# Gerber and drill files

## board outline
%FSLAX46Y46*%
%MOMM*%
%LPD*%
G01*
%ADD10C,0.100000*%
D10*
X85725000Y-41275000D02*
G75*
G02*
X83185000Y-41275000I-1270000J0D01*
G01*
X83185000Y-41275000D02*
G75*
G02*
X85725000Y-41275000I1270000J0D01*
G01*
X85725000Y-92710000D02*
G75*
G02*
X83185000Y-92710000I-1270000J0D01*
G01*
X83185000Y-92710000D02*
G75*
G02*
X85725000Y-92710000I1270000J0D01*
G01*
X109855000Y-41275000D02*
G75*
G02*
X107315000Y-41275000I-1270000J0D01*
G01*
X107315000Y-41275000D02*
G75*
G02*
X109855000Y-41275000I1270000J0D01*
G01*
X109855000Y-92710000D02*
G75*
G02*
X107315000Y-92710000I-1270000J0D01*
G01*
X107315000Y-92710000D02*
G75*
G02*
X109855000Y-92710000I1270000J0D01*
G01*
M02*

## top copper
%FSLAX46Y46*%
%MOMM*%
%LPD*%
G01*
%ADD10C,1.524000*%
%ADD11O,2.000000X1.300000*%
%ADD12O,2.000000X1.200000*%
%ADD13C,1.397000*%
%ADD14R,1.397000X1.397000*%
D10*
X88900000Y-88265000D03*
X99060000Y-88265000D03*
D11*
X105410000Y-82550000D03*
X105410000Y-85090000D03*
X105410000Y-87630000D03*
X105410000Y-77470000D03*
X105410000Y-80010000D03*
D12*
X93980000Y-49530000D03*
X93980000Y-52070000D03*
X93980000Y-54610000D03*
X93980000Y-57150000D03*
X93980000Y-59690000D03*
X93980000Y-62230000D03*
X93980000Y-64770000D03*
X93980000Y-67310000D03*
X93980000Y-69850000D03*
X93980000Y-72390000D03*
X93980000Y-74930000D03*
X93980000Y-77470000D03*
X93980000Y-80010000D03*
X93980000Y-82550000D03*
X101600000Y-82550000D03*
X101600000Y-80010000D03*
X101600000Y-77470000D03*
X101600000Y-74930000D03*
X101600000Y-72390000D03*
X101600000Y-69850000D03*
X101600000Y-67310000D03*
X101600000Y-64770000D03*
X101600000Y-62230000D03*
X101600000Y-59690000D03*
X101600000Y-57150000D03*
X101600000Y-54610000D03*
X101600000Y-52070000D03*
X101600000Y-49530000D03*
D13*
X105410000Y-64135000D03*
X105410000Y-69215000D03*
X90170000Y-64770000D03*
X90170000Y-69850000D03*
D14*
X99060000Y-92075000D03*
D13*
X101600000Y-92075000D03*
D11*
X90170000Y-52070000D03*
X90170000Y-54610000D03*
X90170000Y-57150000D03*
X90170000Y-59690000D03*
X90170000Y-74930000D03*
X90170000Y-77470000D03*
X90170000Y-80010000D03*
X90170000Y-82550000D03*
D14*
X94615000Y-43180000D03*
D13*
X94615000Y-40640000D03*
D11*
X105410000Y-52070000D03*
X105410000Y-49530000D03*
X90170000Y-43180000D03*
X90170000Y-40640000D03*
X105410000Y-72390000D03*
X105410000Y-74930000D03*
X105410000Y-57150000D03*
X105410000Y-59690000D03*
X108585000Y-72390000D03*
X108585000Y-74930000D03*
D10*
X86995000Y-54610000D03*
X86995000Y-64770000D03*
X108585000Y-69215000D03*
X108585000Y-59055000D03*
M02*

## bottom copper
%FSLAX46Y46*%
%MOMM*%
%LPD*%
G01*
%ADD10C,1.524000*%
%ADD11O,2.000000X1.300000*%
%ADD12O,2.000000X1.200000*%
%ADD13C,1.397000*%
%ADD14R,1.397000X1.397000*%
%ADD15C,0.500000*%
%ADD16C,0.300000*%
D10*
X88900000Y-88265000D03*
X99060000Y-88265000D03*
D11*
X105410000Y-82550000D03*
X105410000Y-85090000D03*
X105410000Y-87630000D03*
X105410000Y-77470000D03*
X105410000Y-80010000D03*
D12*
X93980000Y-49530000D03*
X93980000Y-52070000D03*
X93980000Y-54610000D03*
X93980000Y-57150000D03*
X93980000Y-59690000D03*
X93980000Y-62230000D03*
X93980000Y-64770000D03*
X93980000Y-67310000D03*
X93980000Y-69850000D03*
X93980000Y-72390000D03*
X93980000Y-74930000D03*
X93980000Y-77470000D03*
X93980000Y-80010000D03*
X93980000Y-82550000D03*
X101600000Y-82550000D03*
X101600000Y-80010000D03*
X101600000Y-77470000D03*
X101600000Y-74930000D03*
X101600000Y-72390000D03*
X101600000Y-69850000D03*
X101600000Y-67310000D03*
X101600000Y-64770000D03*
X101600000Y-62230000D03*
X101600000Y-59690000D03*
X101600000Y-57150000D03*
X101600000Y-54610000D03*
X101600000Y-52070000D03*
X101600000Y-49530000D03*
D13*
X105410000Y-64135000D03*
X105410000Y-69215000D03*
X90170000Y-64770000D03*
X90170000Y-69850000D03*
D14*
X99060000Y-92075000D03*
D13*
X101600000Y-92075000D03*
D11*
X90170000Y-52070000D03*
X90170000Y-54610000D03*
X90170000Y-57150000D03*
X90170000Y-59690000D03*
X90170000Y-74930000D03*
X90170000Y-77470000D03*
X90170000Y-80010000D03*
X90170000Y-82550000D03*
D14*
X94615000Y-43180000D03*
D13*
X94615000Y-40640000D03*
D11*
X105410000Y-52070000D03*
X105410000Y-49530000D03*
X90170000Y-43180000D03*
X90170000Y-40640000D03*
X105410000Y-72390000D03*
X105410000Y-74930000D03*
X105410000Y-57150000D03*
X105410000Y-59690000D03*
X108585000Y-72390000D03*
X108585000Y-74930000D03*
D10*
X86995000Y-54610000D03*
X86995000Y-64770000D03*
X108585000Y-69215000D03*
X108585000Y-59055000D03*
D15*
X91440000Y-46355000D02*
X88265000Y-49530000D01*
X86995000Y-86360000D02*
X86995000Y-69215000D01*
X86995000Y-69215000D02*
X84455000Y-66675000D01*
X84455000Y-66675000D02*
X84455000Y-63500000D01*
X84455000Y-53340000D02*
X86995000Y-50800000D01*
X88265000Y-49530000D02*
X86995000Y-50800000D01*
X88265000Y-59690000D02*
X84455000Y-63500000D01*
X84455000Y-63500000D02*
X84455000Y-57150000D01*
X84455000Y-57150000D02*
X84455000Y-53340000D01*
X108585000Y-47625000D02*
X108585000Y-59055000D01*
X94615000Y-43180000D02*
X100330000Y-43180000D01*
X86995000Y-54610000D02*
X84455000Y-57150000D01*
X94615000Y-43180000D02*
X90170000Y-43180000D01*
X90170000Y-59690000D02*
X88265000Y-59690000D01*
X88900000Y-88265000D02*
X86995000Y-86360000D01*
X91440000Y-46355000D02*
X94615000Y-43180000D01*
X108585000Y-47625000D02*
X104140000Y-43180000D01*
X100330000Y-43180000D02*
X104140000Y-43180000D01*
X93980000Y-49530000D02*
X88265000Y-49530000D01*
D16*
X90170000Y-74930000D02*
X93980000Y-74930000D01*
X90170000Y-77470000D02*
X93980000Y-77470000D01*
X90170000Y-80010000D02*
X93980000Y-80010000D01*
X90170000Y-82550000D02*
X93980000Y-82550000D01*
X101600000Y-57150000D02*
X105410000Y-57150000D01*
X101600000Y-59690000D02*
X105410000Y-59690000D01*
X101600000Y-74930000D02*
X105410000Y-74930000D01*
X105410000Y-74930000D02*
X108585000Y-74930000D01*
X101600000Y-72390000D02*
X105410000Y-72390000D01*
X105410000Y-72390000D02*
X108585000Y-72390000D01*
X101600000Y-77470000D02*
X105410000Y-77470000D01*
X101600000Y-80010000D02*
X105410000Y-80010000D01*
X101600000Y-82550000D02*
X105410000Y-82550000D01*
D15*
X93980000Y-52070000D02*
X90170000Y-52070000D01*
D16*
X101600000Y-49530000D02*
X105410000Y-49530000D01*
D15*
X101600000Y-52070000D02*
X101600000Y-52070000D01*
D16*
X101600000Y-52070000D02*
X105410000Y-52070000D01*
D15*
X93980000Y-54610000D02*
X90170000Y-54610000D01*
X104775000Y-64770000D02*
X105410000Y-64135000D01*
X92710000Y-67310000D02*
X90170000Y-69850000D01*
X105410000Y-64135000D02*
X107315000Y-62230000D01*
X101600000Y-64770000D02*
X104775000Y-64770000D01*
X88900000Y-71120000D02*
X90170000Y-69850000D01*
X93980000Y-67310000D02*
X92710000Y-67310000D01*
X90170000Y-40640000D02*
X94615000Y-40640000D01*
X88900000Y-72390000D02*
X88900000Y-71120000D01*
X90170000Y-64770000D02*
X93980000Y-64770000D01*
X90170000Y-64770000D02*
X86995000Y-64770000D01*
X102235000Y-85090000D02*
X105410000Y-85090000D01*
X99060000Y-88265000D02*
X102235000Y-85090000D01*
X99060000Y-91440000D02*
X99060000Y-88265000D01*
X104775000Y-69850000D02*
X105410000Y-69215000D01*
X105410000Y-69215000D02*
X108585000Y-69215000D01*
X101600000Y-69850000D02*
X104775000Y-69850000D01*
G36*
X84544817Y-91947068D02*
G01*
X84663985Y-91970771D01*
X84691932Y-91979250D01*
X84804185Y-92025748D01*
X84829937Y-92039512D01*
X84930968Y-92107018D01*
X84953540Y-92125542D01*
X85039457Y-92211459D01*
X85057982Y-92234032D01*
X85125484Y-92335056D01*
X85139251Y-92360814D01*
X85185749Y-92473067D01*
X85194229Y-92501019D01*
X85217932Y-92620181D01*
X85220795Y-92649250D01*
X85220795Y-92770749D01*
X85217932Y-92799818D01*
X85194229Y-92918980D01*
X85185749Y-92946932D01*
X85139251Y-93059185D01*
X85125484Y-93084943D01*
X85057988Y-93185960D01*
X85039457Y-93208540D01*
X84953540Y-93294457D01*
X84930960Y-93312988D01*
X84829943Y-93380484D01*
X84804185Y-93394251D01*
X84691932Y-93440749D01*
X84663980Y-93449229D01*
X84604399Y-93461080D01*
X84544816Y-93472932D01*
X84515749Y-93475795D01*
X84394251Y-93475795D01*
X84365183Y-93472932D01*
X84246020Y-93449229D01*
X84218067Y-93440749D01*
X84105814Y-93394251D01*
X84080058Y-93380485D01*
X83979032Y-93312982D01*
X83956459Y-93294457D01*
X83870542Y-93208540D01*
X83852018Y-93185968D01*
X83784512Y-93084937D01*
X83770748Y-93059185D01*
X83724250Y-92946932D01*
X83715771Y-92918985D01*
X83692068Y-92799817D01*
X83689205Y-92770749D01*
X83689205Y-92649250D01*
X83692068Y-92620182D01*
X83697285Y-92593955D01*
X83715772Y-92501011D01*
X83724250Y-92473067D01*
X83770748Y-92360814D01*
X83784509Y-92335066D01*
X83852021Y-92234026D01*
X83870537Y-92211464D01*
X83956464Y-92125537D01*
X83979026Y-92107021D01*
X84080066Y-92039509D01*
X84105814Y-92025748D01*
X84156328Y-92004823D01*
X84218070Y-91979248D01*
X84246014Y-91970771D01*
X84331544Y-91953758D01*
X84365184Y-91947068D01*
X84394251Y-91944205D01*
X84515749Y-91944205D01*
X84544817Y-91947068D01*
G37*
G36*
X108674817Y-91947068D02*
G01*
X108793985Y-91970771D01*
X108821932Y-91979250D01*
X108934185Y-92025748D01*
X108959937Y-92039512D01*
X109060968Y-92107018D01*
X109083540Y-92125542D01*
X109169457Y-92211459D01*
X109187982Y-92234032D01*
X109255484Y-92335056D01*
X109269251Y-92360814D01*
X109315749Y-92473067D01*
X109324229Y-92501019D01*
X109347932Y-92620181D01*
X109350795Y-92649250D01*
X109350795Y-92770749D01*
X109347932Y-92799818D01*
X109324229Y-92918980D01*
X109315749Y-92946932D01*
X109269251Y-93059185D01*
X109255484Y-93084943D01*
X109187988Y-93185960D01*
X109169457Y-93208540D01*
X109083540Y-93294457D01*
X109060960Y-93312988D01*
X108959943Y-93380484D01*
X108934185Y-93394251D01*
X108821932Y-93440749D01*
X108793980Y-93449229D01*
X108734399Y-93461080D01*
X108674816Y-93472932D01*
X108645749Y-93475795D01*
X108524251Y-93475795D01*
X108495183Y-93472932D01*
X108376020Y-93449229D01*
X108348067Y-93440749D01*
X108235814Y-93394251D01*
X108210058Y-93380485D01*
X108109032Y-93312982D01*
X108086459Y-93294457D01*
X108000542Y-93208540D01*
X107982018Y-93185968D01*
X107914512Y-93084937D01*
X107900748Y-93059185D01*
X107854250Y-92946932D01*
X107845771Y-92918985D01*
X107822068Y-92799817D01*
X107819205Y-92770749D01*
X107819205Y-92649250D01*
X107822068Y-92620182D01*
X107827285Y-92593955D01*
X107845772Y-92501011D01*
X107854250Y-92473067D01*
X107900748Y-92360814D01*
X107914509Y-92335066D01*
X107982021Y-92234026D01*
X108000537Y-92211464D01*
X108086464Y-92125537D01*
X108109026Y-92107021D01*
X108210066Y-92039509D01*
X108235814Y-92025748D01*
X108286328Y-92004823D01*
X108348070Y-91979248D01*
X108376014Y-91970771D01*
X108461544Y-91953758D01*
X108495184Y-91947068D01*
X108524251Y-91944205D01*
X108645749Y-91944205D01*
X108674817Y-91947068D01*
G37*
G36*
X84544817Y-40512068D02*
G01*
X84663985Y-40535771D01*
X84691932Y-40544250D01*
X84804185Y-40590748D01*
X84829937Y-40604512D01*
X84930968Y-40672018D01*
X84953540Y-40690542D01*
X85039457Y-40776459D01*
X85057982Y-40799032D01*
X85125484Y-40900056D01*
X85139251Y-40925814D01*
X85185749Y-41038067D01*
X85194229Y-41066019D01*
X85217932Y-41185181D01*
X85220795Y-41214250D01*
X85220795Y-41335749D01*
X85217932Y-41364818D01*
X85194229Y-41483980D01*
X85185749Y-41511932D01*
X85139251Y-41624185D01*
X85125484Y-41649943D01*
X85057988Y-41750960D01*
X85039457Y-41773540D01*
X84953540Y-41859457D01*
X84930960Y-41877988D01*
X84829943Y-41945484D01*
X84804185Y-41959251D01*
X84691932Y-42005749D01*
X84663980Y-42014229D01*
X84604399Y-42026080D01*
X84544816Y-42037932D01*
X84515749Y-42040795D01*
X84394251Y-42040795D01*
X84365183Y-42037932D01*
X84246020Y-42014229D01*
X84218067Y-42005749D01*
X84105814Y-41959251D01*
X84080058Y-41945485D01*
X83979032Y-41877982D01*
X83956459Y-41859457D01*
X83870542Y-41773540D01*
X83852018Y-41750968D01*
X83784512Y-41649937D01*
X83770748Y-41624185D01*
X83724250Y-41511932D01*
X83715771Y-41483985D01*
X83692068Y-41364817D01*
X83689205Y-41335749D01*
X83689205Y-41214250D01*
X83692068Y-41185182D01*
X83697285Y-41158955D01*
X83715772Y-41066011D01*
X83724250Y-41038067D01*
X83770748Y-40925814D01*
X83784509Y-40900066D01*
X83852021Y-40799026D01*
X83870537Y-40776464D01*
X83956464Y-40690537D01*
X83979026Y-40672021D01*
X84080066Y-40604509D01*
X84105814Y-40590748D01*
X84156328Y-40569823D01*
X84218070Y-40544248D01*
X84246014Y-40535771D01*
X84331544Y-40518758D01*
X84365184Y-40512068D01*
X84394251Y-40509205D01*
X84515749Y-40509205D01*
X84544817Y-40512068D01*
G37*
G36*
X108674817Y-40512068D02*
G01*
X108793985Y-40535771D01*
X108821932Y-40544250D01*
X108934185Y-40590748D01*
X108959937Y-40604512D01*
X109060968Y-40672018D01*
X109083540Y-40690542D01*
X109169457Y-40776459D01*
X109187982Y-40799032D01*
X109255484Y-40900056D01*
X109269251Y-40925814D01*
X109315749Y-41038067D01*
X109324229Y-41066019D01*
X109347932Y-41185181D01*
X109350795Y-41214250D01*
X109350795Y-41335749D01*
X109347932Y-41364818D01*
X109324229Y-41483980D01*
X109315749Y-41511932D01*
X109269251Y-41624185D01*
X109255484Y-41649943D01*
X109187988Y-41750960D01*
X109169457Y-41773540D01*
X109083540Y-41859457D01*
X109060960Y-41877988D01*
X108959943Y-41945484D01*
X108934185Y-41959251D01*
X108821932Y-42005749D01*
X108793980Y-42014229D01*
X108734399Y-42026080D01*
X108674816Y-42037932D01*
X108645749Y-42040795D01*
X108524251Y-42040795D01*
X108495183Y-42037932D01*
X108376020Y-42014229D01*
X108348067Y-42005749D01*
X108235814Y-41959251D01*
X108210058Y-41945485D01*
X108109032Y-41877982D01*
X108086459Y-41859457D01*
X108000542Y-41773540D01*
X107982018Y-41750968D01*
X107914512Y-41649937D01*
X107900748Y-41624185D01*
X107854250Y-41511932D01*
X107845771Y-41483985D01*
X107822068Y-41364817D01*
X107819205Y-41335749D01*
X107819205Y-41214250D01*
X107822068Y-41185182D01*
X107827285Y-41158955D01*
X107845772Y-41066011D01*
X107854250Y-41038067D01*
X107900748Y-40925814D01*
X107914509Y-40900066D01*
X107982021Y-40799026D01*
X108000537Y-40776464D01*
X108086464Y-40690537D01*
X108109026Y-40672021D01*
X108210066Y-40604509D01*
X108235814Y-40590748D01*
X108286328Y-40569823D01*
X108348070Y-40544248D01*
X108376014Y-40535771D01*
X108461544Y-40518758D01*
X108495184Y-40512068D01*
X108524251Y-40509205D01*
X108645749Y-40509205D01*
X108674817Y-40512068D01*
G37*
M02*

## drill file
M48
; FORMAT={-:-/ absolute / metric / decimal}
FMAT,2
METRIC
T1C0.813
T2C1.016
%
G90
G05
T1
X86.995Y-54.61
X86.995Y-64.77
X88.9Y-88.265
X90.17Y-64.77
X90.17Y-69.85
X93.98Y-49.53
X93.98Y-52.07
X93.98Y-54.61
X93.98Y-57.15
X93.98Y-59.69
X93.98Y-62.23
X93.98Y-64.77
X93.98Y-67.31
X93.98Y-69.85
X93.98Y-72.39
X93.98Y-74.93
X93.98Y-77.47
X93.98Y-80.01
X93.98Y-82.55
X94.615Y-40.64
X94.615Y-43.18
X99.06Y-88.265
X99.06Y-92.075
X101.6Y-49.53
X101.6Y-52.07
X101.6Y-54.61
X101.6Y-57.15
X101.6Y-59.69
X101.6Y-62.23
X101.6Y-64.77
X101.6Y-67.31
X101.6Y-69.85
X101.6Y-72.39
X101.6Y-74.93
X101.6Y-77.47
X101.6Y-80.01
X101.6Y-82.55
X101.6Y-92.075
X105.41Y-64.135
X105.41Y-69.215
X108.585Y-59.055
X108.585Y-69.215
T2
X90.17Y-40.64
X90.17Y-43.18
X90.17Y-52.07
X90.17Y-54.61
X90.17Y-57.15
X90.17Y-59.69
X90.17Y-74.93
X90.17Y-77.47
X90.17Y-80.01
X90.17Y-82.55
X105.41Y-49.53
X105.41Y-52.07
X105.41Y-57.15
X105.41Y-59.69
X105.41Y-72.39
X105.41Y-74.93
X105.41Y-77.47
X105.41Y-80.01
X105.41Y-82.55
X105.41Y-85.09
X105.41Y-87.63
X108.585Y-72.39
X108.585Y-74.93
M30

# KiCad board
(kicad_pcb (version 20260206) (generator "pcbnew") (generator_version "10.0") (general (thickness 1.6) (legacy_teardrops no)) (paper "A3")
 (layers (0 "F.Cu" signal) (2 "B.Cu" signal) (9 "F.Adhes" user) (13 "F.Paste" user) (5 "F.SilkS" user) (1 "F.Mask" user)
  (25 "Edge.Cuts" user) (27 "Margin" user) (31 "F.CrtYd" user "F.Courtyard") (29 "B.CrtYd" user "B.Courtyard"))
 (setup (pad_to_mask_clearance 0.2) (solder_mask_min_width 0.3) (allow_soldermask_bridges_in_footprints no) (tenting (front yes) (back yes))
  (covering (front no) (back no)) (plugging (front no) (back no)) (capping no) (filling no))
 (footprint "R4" (layer "F.Cu") (at 93.98 88.265)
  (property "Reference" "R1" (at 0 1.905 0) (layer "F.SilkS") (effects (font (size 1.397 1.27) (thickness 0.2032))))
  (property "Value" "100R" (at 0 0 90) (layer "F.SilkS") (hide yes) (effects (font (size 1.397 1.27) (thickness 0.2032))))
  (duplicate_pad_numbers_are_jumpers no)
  (pad "1" thru_hole circle (at -5.08 0) (size 1.524 1.524) (drill 0.8128) (layers "*.Cu" "*.Mask" "F.SilkS") (remove_unused_layers no)
   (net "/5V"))
  (pad "2" thru_hole circle (at 5.08 0) (size 1.524 1.524) (drill 0.8128) (layers "*.Cu" "*.Mask" "F.SilkS") (remove_unused_layers no)
   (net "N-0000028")))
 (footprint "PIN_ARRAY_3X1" (layer "F.Cu") (at 105.41 85.09 -90)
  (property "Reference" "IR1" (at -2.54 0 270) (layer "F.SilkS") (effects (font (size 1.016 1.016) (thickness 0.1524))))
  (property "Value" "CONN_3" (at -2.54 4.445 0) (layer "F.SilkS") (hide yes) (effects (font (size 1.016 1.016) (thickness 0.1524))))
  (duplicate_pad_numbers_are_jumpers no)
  (pad "1" thru_hole oval (at -2.54 0 270) (size 1.3 2) (drill 1.016) (layers "*.Cu" "*.Mask" "F.SilkS") (remove_unused_layers no)
   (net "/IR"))
  (pad "2" thru_hole oval (at 0 0 270) (size 1.3 2) (drill 1.016) (layers "*.Cu" "*.Mask" "F.SilkS") (remove_unused_layers no)
   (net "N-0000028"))
  (pad "3" thru_hole oval (at 2.54 0 270) (size 1.3 2) (drill 1.016) (layers "*.Cu" "*.Mask" "F.SilkS") (remove_unused_layers no)
   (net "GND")))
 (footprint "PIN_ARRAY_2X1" (layer "F.Cu") (at 105.41 78.74 -90)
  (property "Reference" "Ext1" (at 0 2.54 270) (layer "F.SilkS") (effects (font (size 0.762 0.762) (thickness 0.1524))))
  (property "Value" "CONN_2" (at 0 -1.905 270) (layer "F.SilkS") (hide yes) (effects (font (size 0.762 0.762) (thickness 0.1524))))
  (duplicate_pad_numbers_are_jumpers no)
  (pad "1" thru_hole oval (at -1.27 0 270) (size 1.3 2) (drill 1.016) (layers "*.Cu" "*.Mask" "F.SilkS") (remove_unused_layers no)
   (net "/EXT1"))
  (pad "2" thru_hole oval (at 1.27 0 270) (size 1.3 2) (drill 1.016) (layers "*.Cu" "*.Mask" "F.SilkS") (remove_unused_layers no)
   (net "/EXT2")))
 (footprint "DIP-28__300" (layer "F.Cu") (at 97.79 66.04 -90)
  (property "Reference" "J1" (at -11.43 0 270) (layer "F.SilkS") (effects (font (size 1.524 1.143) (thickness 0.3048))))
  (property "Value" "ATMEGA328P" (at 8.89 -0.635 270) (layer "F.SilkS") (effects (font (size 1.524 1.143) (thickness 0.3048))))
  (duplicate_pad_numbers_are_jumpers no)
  (pad "1" thru_hole oval (at -16.51 3.81 270) (size 1.2 2) (drill 0.8128) (layers "*.Cu" "*.Mask" "F.SilkS") (remove_unused_layers no)
   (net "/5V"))
  (pad "2" thru_hole oval (at -13.97 3.81 270) (size 1.2 2) (drill 0.8128) (layers "*.Cu" "*.Mask" "F.SilkS") (remove_unused_layers no)
   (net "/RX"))
  (pad "3" thru_hole oval (at -11.43 3.81 270) (size 1.2 2) (drill 0.8128) (layers "*.Cu" "*.Mask" "F.SilkS") (remove_unused_layers no)
   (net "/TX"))
  (pad "4" thru_hole oval (at -8.89 3.81 270) (size 1.2 2) (drill 0.8128) (layers "*.Cu" "*.Mask" "F.SilkS") (remove_unused_layers no))
  (pad "5" thru_hole oval (at -6.35 3.81 270) (size 1.2 2) (drill 0.8128) (layers "*.Cu" "*.Mask" "F.SilkS") (remove_unused_layers no))
  (pad "6" thru_hole oval (at -3.81 3.81 270) (size 1.2 2) (drill 0.8128) (layers "*.Cu" "*.Mask" "F.SilkS") (remove_unused_layers no))
  (pad "7" thru_hole oval (at -1.27 3.81 270) (size 1.2 2) (drill 0.8128) (layers "*.Cu" "*.Mask" "F.SilkS") (remove_unused_layers no)
   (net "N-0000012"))
  (pad "8" thru_hole oval (at 1.27 3.81 270) (size 1.2 2) (drill 0.8128) (layers "*.Cu" "*.Mask" "F.SilkS") (remove_unused_layers no)
   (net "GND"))
  (pad "9" thru_hole oval (at 3.81 3.81 270) (size 1.2 2) (drill 0.8128) (layers "*.Cu" "*.Mask" "F.SilkS") (remove_unused_layers no))
  (pad "10" thru_hole oval (at 6.35 3.81 270) (size 1.2 2) (drill 0.8128) (layers "*.Cu" "*.Mask" "F.SilkS") (remove_unused_layers no))
  (pad "11" thru_hole oval (at 8.89 3.81 270) (size 1.2 2) (drill 0.8128) (layers "*.Cu" "*.Mask" "F.SilkS") (remove_unused_layers no)
   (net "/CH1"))
  (pad "12" thru_hole oval (at 11.43 3.81 270) (size 1.2 2) (drill 0.8128) (layers "*.Cu" "*.Mask" "F.SilkS") (remove_unused_layers no)
   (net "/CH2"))
  (pad "13" thru_hole oval (at 13.97 3.81 270) (size 1.2 2) (drill 0.8128) (layers "*.Cu" "*.Mask" "F.SilkS") (remove_unused_layers no)
   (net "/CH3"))
  (pad "14" thru_hole oval (at 16.51 3.81 270) (size 1.2 2) (drill 0.8128) (layers "*.Cu" "*.Mask" "F.SilkS") (remove_unused_layers no)
   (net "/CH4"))
  (pad "15" thru_hole oval (at 16.51 -3.81 270) (size 1.2 2) (drill 0.8128) (layers "*.Cu" "*.Mask" "F.SilkS") (remove_unused_layers no)
   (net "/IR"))
  (pad "16" thru_hole oval (at 13.97 -3.81 270) (size 1.2 2) (drill 0.8128) (layers "*.Cu" "*.Mask" "F.SilkS") (remove_unused_layers no)
   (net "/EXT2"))
  (pad "17" thru_hole oval (at 11.43 -3.81 270) (size 1.2 2) (drill 0.8128) (layers "*.Cu" "*.Mask" "F.SilkS") (remove_unused_layers no)
   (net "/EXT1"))
  (pad "18" thru_hole oval (at 8.89 -3.81 270) (size 1.2 2) (drill 0.8128) (layers "*.Cu" "*.Mask" "F.SilkS") (remove_unused_layers no)
   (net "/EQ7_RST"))
  (pad "19" thru_hole oval (at 6.35 -3.81 270) (size 1.2 2) (drill 0.8128) (layers "*.Cu" "*.Mask" "F.SilkS") (remove_unused_layers no)
   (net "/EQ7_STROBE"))
  (pad "20" thru_hole oval (at 3.81 -3.81 270) (size 1.2 2) (drill 0.8128) (layers "*.Cu" "*.Mask" "F.SilkS") (remove_unused_layers no)
   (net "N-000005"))
  (pad "21" thru_hole oval (at 1.27 -3.81 270) (size 1.2 2) (drill 0.8128) (layers "*.Cu" "*.Mask" "F.SilkS") (remove_unused_layers no))
  (pad "22" thru_hole oval (at -1.27 -3.81 270) (size 1.2 2) (drill 0.8128) (layers "*.Cu" "*.Mask" "F.SilkS") (remove_unused_layers no)
   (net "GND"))
  (pad "23" thru_hole oval (at -3.81 -3.81 270) (size 1.2 2) (drill 0.8128) (layers "*.Cu" "*.Mask" "F.SilkS") (remove_unused_layers no))
  (pad "24" thru_hole oval (at -6.35 -3.81 270) (size 1.2 2) (drill 0.8128) (layers "*.Cu" "*.Mask" "F.SilkS") (remove_unused_layers no)
   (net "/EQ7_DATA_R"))
  (pad "25" thru_hole oval (at -8.89 -3.81 270) (size 1.2 2) (drill 0.8128) (layers "*.Cu" "*.Mask" "F.SilkS") (remove_unused_layers no)
   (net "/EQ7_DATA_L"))
  (pad "26" thru_hole oval (at -11.43 -3.81 270) (size 1.2 2) (drill 0.8128) (layers "*.Cu" "*.Mask" "F.SilkS") (remove_unused_layers no))
  (pad "27" thru_hole oval (at -13.97 -3.81 270) (size 1.2 2) (drill 0.8128) (layers "*.Cu" "*.Mask" "F.SilkS") (remove_unused_layers no)
   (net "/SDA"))
  (pad "28" thru_hole oval (at -16.51 -3.81 270) (size 1.2 2) (drill 0.8128) (layers "*.Cu" "*.Mask" "F.SilkS") (remove_unused_layers no)
   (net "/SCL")))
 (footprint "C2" (layer "F.Cu") (at 105.41 66.675 -90)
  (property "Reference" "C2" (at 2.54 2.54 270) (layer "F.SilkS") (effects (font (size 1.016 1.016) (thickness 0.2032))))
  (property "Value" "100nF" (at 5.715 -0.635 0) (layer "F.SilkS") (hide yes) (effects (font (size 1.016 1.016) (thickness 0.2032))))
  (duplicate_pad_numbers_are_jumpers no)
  (pad "1" thru_hole circle (at -2.54 0 270) (size 1.397 1.397) (drill 0.8128) (layers "*.Cu" "*.Mask" "F.SilkS") (remove_unused_layers no)
   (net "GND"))
  (pad "2" thru_hole circle (at 2.54 0 270) (size 1.397 1.397) (drill 0.8128) (layers "*.Cu" "*.Mask" "F.SilkS") (remove_unused_layers no)
   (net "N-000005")))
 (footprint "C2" (layer "F.Cu") (at 90.17 67.31 -90)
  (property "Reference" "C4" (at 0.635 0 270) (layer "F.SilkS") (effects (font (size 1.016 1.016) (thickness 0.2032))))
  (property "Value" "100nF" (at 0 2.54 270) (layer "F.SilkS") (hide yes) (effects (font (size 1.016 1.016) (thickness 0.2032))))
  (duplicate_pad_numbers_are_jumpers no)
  (pad "1" thru_hole circle (at -2.54 0 270) (size 1.397 1.397) (drill 0.8128) (layers "*.Cu" "*.Mask" "F.SilkS") (remove_unused_layers no)
   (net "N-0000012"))
  (pad "2" thru_hole circle (at 2.54 0 270) (size 1.397 1.397) (drill 0.8128) (layers "*.Cu" "*.Mask" "F.SilkS") (remove_unused_layers no)
   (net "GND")))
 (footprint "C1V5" (layer "F.Cu") (at 100.33 92.075)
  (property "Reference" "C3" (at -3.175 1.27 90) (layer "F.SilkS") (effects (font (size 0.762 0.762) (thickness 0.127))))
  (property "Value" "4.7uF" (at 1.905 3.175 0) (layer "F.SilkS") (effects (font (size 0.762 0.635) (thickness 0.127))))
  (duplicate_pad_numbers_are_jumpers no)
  (pad "1" thru_hole rect (at -1.27 0) (size 1.397 1.397) (drill 0.8128) (layers "*.Cu" "*.Mask" "F.SilkS") (remove_unused_layers no)
   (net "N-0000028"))
  (pad "2" thru_hole circle (at 1.27 0) (size 1.397 1.397) (drill 0.8128) (layers "*.Cu" "*.Mask" "F.SilkS") (remove_unused_layers no)
   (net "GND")))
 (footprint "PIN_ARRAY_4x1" (layer "F.Cu") (at 90.17 55.88 -90)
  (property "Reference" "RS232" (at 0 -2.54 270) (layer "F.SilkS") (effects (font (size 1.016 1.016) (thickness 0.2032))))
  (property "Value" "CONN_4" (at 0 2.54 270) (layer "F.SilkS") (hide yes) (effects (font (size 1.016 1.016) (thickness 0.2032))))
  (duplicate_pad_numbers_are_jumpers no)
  (pad "1" thru_hole oval (at -3.81 0 270) (size 1.3 2) (drill 1.016) (layers "*.Cu" "*.Mask" "F.SilkS") (remove_unused_layers no)
   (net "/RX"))
  (pad "2" thru_hole oval (at -1.27 0 270) (size 1.3 2) (drill 1.016) (layers "*.Cu" "*.Mask" "F.SilkS") (remove_unused_layers no)
   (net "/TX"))
  (pad "3" thru_hole oval (at 1.27 0 270) (size 1.3 2) (drill 1.016) (layers "*.Cu" "*.Mask" "F.SilkS") (remove_unused_layers no)
   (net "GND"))
  (pad "4" thru_hole oval (at 3.81 0 270) (size 1.3 2) (drill 1.016) (layers "*.Cu" "*.Mask" "F.SilkS") (remove_unused_layers no)
   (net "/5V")))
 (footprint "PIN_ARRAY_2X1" (layer "F.Cu") (at 90.17 76.2 -90)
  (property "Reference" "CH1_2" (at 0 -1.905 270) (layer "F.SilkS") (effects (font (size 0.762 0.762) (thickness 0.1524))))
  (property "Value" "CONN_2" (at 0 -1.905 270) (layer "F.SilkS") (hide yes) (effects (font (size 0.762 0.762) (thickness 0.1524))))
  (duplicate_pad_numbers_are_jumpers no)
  (pad "1" thru_hole oval (at -1.27 0 270) (size 1.3 2) (drill 1.016) (layers "*.Cu" "*.Mask" "F.SilkS") (remove_unused_layers no)
   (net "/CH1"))
  (pad "2" thru_hole oval (at 1.27 0 270) (size 1.3 2) (drill 1.016) (layers "*.Cu" "*.Mask" "F.SilkS") (remove_unused_layers no)
   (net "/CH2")))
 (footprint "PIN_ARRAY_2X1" (layer "F.Cu") (at 90.17 81.28 -90)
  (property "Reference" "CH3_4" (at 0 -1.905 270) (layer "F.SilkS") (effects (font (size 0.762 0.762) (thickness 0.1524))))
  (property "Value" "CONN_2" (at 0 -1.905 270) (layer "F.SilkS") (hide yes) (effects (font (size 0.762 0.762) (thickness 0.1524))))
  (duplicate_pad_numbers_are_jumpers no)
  (pad "1" thru_hole oval (at -1.27 0 270) (size 1.3 2) (drill 1.016) (layers "*.Cu" "*.Mask" "F.SilkS") (remove_unused_layers no)
   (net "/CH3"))
  (pad "2" thru_hole oval (at 1.27 0 270) (size 1.3 2) (drill 1.016) (layers "*.Cu" "*.Mask" "F.SilkS") (remove_unused_layers no)
   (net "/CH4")))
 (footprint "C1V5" (layer "F.Cu") (at 94.615 41.91 90)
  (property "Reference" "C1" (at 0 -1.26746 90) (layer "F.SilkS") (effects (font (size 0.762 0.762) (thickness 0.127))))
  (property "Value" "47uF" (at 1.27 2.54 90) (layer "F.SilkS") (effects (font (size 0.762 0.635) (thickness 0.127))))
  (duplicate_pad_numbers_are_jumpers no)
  (pad "1" thru_hole rect (at -1.27 0 90) (size 1.397 1.397) (drill 0.8128) (layers "*.Cu" "*.Mask" "F.SilkS") (remove_unused_layers no)
   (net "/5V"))
  (pad "2" thru_hole circle (at 1.27 0 90) (size 1.397 1.397) (drill 0.8128) (layers "*.Cu" "*.Mask" "F.SilkS") (remove_unused_layers no)
   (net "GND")))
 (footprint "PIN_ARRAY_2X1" (layer "F.Cu") (at 105.41 50.8 90)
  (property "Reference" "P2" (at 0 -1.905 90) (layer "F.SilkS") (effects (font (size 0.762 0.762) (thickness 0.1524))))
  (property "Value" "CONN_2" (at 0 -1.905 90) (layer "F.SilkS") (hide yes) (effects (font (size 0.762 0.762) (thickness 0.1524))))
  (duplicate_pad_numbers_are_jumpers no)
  (pad "1" thru_hole oval (at -1.27 0 90) (size 1.3 2) (drill 1.016) (layers "*.Cu" "*.Mask" "F.SilkS") (remove_unused_layers no)
   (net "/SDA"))
  (pad "2" thru_hole oval (at 1.27 0 90) (size 1.3 2) (drill 1.016) (layers "*.Cu" "*.Mask" "F.SilkS") (remove_unused_layers no)
   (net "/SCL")))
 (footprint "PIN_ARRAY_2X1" (layer "F.Cu") (at 90.17 41.91 90)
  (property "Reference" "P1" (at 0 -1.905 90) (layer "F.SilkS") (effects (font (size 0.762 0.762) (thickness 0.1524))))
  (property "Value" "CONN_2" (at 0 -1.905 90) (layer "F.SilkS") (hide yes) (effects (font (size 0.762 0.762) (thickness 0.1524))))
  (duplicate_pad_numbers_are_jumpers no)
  (pad "1" thru_hole oval (at -1.27 0 90) (size 1.3 2) (drill 1.016) (layers "*.Cu" "*.Mask" "F.SilkS") (remove_unused_layers no)
   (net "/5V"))
  (pad "2" thru_hole oval (at 1.27 0 90) (size 1.3 2) (drill 1.016) (layers "*.Cu" "*.Mask" "F.SilkS") (remove_unused_layers no) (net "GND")))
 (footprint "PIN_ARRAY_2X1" (layer "F.Cu") (at 105.41 73.66 -90)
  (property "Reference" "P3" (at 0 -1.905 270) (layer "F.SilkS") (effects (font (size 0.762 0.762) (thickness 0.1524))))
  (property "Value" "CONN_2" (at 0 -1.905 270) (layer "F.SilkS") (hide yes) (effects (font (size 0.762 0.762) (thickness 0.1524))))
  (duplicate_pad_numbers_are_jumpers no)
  (pad "1" thru_hole oval (at -1.27 0 270) (size 1.3 2) (drill 1.016) (layers "*.Cu" "*.Mask" "F.SilkS") (remove_unused_layers no)
   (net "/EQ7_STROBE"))
  (pad "2" thru_hole oval (at 1.27 0 270) (size 1.3 2) (drill 1.016) (layers "*.Cu" "*.Mask" "F.SilkS") (remove_unused_layers no)
   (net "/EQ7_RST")))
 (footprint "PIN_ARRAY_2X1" (layer "F.Cu") (at 105.41 58.42 -90)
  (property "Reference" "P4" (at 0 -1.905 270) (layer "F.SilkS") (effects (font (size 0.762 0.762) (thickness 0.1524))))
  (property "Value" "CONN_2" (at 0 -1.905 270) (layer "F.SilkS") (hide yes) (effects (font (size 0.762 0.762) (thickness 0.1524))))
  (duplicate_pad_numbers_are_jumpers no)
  (pad "1" thru_hole oval (at -1.27 0 270) (size 1.3 2) (drill 1.016) (layers "*.Cu" "*.Mask" "F.SilkS") (remove_unused_layers no)
   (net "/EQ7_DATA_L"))
  (pad "2" thru_hole oval (at 1.27 0 270) (size 1.3 2) (drill 1.016) (layers "*.Cu" "*.Mask" "F.SilkS") (remove_unused_layers no)
   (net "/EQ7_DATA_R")))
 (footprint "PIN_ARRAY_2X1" (layer "F.Cu") (at 108.585 73.66 -90)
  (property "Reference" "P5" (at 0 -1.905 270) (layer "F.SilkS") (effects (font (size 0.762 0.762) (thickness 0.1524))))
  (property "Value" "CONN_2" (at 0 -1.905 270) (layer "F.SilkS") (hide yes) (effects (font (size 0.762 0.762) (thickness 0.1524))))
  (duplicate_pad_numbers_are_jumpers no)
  (pad "1" thru_hole oval (at -1.27 0 270) (size 1.3 2) (drill 1.016) (layers "*.Cu" "*.Mask" "F.SilkS") (remove_unused_layers no)
   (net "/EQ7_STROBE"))
  (pad "2" thru_hole oval (at 1.27 0 270) (size 1.3 2) (drill 1.016) (layers "*.Cu" "*.Mask" "F.SilkS") (remove_unused_layers no)
   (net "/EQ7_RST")))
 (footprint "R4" (layer "F.Cu") (at 86.995 59.69 -90)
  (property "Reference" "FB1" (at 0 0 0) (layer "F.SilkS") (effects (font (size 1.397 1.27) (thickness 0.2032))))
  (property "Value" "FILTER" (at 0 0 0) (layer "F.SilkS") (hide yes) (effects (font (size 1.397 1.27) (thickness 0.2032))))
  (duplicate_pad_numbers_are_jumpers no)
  (pad "1" thru_hole circle (at -5.08 0 270) (size 1.524 1.524) (drill 0.8128) (layers "*.Cu" "*.Mask" "F.SilkS") (remove_unused_layers no)
   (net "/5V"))
  (pad "2" thru_hole circle (at 5.08 0 270) (size 1.524 1.524) (drill 0.8128) (layers "*.Cu" "*.Mask" "F.SilkS") (remove_unused_layers no)
   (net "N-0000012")))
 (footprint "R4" (layer "F.Cu") (at 108.585 64.135 90)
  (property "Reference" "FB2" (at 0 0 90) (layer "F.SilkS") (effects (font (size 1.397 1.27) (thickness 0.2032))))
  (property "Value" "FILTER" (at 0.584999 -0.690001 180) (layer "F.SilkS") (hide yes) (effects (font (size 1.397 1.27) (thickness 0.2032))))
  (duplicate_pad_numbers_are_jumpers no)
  (pad "1" thru_hole circle (at -5.08 0 90) (size 1.524 1.524) (drill 0.8128) (layers "*.Cu" "*.Mask" "F.SilkS") (remove_unused_layers no)
   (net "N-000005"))
  (pad "2" thru_hole circle (at 5.08 0 90) (size 1.524 1.524) (drill 0.8128) (layers "*.Cu" "*.Mask" "F.SilkS") (remove_unused_layers no)
   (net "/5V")))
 (gr_circle (center 84.455 41.275) (end 85.725 41.275) (stroke (width 0.1) (type solid)) (fill no) (layer "Edge.Cuts"))
 (gr_circle (center 84.455 92.71) (end 85.725 92.71) (stroke (width 0.1) (type solid)) (fill no) (layer "Edge.Cuts"))
 (gr_circle (center 108.585 41.275) (end 109.855 41.275) (stroke (width 0.1) (type solid)) (fill no) (layer "Edge.Cuts"))
 (gr_circle (center 108.585 92.71) (end 109.855 92.71) (stroke (width 0.1) (type solid)) (fill no) (layer "Edge.Cuts"))
 (segment (start 91.44 46.355) (end 88.265 49.53) (width 0.5) (layer "B.Cu") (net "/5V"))
 (segment (start 86.995 86.36) (end 86.995 69.215) (width 0.5) (layer "B.Cu") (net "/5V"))
 (segment (start 86.995 69.215) (end 84.455 66.675) (width 0.5) (layer "B.Cu") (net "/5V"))
 (segment (start 84.455 66.675) (end 84.455 63.5) (width 0.5) (layer "B.Cu") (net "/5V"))
 (segment (start 84.455 53.34) (end 86.995 50.8) (width 0.5) (layer "B.Cu") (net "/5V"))
 (segment (start 88.265 49.53) (end 86.995 50.8) (width 0.5) (layer "B.Cu") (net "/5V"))
 (segment (start 88.265 59.69) (end 84.455 63.5) (width 0.5) (layer "B.Cu") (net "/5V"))
 (segment (start 84.455 63.5) (end 84.455 57.15) (width 0.5) (layer "B.Cu") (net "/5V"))
 (segment (start 84.455 57.15) (end 84.455 53.34) (width 0.5) (layer "B.Cu") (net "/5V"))
 (segment (start 108.585 47.625) (end 108.585 59.055) (width 0.5) (layer "B.Cu") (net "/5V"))
 (segment (start 94.615 43.18) (end 100.33 43.18) (width 0.5) (layer "B.Cu") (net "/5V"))
 (segment (start 86.995 54.61) (end 84.455 57.15) (width 0.5) (layer "B.Cu") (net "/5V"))
 (segment (start 94.615 43.18) (end 90.17 43.18) (width 0.5) (layer "B.Cu") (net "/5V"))
 (segment (start 90.17 59.69) (end 88.265 59.69) (width 0.5) (layer "B.Cu") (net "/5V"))
 (segment (start 88.9 88.265) (end 86.995 86.36) (width 0.5) (layer "B.Cu") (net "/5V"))
 (segment (start 91.44 46.355) (end 94.615 43.18) (width 0.5) (layer "B.Cu") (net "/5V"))
 (segment (start 108.585 47.625) (end 104.14 43.18) (width 0.5) (layer "B.Cu") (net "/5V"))
 (segment (start 100.33 43.18) (end 104.14 43.18) (width 0.5) (layer "B.Cu") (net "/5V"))
 (segment (start 93.98 49.53) (end 88.265 49.53) (width 0.5) (layer "B.Cu") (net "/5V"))
 (segment (start 90.17 74.93) (end 93.98 74.93) (width 0.3) (layer "B.Cu") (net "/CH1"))
 (segment (start 90.17 77.47) (end 93.98 77.47) (width 0.3) (layer "B.Cu") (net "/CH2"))
 (segment (start 90.17 80.01) (end 93.98 80.01) (width 0.3) (layer "B.Cu") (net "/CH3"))
 (segment (start 90.17 82.55) (end 93.98 82.55) (width 0.3) (layer "B.Cu") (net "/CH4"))
 (segment (start 101.6 57.15) (end 105.41 57.15) (width 0.3) (layer "B.Cu") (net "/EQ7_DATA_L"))
 (segment (start 101.6 59.69) (end 105.41 59.69) (width 0.3) (layer "B.Cu") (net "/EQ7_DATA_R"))
 (segment (start 101.6 74.93) (end 105.41 74.93) (width 0.3) (layer "B.Cu") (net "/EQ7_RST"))
 (segment (start 105.41 74.93) (end 108.585 74.93) (width 0.3) (layer "B.Cu") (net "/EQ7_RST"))
 (segment (start 101.6 72.39) (end 105.41 72.39) (width 0.3) (layer "B.Cu") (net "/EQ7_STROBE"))
 (segment (start 105.41 72.39) (end 108.585 72.39) (width 0.3) (layer "B.Cu") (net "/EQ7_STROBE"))
 (segment (start 101.6 77.47) (end 105.41 77.47) (width 0.3) (layer "B.Cu") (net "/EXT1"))
 (segment (start 101.6 80.01) (end 105.41 80.01) (width 0.3) (layer "B.Cu") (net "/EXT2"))
 (segment (start 101.6 82.55) (end 105.41 82.55) (width 0.3) (layer "B.Cu") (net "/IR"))
 (segment (start 93.98 52.07) (end 90.17 52.07) (width 0.5) (layer "B.Cu") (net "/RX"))
 (segment (start 101.6 49.53) (end 105.41 49.53) (width 0.3) (layer "B.Cu") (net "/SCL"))
 (segment (start 101.6 52.07) (end 101.6 52.07) (width 0.5) (layer "B.Cu") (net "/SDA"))
 (segment (start 101.6 52.07) (end 105.41 52.07) (width 0.3) (layer "B.Cu") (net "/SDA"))
 (segment (start 93.98 54.61) (end 90.17 54.61) (width 0.5) (layer "B.Cu") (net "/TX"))
 (segment (start 104.775 64.77) (end 105.41 64.135) (width 0.5) (layer "B.Cu") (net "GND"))
 (segment (start 92.71 67.31) (end 90.17 69.85) (width 0.5) (layer "B.Cu") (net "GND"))
 (segment (start 105.41 64.135) (end 107.315 62.23) (width 0.5) (layer "B.Cu") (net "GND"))
 (segment (start 101.6 64.77) (end 104.775 64.77) (width 0.5) (layer "B.Cu") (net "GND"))
 (segment (start 88.9 71.12) (end 90.17 69.85) (width 0.5) (layer "B.Cu") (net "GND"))
 (segment (start 93.98 67.31) (end 92.71 67.31) (width 0.5) (layer "B.Cu") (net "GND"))
 (segment (start 90.17 40.64) (end 94.615 40.64) (width 0.5) (layer "B.Cu") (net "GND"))
 (segment (start 88.9 72.39) (end 88.9 71.12) (width 0.5) (layer "B.Cu") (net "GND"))
 (segment (start 90.17 64.77) (end 93.98 64.77) (width 0.5) (layer "B.Cu") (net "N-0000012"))
 (segment (start 90.17 64.77) (end 86.995 64.77) (width 0.5) (layer "B.Cu") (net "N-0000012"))
 (segment (start 102.235 85.09) (end 105.41 85.09) (width 0.5) (layer "B.Cu") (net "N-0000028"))
 (segment (start 99.06 88.265) (end 102.235 85.09) (width 0.5) (layer "B.Cu") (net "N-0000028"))
 (segment (start 99.06 91.44) (end 99.06 88.265) (width 0.5) (layer "B.Cu") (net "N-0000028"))
 (segment (start 104.775 69.85) (end 105.41 69.215) (width 0.5) (layer "B.Cu") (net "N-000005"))
 (segment (start 105.41 69.215) (end 108.585 69.215) (width 0.5) (layer "B.Cu") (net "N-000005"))
 (segment (start 101.6 69.85) (end 104.775 69.85) (width 0.5) (layer "B.Cu") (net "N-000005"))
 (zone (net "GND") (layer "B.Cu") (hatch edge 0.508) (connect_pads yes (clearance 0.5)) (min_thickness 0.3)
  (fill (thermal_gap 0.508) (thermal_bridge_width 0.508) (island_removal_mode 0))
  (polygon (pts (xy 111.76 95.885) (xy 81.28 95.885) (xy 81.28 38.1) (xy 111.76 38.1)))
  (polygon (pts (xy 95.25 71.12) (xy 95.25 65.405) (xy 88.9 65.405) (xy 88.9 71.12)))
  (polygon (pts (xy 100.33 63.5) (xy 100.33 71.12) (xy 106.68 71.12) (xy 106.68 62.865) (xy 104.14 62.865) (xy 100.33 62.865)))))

